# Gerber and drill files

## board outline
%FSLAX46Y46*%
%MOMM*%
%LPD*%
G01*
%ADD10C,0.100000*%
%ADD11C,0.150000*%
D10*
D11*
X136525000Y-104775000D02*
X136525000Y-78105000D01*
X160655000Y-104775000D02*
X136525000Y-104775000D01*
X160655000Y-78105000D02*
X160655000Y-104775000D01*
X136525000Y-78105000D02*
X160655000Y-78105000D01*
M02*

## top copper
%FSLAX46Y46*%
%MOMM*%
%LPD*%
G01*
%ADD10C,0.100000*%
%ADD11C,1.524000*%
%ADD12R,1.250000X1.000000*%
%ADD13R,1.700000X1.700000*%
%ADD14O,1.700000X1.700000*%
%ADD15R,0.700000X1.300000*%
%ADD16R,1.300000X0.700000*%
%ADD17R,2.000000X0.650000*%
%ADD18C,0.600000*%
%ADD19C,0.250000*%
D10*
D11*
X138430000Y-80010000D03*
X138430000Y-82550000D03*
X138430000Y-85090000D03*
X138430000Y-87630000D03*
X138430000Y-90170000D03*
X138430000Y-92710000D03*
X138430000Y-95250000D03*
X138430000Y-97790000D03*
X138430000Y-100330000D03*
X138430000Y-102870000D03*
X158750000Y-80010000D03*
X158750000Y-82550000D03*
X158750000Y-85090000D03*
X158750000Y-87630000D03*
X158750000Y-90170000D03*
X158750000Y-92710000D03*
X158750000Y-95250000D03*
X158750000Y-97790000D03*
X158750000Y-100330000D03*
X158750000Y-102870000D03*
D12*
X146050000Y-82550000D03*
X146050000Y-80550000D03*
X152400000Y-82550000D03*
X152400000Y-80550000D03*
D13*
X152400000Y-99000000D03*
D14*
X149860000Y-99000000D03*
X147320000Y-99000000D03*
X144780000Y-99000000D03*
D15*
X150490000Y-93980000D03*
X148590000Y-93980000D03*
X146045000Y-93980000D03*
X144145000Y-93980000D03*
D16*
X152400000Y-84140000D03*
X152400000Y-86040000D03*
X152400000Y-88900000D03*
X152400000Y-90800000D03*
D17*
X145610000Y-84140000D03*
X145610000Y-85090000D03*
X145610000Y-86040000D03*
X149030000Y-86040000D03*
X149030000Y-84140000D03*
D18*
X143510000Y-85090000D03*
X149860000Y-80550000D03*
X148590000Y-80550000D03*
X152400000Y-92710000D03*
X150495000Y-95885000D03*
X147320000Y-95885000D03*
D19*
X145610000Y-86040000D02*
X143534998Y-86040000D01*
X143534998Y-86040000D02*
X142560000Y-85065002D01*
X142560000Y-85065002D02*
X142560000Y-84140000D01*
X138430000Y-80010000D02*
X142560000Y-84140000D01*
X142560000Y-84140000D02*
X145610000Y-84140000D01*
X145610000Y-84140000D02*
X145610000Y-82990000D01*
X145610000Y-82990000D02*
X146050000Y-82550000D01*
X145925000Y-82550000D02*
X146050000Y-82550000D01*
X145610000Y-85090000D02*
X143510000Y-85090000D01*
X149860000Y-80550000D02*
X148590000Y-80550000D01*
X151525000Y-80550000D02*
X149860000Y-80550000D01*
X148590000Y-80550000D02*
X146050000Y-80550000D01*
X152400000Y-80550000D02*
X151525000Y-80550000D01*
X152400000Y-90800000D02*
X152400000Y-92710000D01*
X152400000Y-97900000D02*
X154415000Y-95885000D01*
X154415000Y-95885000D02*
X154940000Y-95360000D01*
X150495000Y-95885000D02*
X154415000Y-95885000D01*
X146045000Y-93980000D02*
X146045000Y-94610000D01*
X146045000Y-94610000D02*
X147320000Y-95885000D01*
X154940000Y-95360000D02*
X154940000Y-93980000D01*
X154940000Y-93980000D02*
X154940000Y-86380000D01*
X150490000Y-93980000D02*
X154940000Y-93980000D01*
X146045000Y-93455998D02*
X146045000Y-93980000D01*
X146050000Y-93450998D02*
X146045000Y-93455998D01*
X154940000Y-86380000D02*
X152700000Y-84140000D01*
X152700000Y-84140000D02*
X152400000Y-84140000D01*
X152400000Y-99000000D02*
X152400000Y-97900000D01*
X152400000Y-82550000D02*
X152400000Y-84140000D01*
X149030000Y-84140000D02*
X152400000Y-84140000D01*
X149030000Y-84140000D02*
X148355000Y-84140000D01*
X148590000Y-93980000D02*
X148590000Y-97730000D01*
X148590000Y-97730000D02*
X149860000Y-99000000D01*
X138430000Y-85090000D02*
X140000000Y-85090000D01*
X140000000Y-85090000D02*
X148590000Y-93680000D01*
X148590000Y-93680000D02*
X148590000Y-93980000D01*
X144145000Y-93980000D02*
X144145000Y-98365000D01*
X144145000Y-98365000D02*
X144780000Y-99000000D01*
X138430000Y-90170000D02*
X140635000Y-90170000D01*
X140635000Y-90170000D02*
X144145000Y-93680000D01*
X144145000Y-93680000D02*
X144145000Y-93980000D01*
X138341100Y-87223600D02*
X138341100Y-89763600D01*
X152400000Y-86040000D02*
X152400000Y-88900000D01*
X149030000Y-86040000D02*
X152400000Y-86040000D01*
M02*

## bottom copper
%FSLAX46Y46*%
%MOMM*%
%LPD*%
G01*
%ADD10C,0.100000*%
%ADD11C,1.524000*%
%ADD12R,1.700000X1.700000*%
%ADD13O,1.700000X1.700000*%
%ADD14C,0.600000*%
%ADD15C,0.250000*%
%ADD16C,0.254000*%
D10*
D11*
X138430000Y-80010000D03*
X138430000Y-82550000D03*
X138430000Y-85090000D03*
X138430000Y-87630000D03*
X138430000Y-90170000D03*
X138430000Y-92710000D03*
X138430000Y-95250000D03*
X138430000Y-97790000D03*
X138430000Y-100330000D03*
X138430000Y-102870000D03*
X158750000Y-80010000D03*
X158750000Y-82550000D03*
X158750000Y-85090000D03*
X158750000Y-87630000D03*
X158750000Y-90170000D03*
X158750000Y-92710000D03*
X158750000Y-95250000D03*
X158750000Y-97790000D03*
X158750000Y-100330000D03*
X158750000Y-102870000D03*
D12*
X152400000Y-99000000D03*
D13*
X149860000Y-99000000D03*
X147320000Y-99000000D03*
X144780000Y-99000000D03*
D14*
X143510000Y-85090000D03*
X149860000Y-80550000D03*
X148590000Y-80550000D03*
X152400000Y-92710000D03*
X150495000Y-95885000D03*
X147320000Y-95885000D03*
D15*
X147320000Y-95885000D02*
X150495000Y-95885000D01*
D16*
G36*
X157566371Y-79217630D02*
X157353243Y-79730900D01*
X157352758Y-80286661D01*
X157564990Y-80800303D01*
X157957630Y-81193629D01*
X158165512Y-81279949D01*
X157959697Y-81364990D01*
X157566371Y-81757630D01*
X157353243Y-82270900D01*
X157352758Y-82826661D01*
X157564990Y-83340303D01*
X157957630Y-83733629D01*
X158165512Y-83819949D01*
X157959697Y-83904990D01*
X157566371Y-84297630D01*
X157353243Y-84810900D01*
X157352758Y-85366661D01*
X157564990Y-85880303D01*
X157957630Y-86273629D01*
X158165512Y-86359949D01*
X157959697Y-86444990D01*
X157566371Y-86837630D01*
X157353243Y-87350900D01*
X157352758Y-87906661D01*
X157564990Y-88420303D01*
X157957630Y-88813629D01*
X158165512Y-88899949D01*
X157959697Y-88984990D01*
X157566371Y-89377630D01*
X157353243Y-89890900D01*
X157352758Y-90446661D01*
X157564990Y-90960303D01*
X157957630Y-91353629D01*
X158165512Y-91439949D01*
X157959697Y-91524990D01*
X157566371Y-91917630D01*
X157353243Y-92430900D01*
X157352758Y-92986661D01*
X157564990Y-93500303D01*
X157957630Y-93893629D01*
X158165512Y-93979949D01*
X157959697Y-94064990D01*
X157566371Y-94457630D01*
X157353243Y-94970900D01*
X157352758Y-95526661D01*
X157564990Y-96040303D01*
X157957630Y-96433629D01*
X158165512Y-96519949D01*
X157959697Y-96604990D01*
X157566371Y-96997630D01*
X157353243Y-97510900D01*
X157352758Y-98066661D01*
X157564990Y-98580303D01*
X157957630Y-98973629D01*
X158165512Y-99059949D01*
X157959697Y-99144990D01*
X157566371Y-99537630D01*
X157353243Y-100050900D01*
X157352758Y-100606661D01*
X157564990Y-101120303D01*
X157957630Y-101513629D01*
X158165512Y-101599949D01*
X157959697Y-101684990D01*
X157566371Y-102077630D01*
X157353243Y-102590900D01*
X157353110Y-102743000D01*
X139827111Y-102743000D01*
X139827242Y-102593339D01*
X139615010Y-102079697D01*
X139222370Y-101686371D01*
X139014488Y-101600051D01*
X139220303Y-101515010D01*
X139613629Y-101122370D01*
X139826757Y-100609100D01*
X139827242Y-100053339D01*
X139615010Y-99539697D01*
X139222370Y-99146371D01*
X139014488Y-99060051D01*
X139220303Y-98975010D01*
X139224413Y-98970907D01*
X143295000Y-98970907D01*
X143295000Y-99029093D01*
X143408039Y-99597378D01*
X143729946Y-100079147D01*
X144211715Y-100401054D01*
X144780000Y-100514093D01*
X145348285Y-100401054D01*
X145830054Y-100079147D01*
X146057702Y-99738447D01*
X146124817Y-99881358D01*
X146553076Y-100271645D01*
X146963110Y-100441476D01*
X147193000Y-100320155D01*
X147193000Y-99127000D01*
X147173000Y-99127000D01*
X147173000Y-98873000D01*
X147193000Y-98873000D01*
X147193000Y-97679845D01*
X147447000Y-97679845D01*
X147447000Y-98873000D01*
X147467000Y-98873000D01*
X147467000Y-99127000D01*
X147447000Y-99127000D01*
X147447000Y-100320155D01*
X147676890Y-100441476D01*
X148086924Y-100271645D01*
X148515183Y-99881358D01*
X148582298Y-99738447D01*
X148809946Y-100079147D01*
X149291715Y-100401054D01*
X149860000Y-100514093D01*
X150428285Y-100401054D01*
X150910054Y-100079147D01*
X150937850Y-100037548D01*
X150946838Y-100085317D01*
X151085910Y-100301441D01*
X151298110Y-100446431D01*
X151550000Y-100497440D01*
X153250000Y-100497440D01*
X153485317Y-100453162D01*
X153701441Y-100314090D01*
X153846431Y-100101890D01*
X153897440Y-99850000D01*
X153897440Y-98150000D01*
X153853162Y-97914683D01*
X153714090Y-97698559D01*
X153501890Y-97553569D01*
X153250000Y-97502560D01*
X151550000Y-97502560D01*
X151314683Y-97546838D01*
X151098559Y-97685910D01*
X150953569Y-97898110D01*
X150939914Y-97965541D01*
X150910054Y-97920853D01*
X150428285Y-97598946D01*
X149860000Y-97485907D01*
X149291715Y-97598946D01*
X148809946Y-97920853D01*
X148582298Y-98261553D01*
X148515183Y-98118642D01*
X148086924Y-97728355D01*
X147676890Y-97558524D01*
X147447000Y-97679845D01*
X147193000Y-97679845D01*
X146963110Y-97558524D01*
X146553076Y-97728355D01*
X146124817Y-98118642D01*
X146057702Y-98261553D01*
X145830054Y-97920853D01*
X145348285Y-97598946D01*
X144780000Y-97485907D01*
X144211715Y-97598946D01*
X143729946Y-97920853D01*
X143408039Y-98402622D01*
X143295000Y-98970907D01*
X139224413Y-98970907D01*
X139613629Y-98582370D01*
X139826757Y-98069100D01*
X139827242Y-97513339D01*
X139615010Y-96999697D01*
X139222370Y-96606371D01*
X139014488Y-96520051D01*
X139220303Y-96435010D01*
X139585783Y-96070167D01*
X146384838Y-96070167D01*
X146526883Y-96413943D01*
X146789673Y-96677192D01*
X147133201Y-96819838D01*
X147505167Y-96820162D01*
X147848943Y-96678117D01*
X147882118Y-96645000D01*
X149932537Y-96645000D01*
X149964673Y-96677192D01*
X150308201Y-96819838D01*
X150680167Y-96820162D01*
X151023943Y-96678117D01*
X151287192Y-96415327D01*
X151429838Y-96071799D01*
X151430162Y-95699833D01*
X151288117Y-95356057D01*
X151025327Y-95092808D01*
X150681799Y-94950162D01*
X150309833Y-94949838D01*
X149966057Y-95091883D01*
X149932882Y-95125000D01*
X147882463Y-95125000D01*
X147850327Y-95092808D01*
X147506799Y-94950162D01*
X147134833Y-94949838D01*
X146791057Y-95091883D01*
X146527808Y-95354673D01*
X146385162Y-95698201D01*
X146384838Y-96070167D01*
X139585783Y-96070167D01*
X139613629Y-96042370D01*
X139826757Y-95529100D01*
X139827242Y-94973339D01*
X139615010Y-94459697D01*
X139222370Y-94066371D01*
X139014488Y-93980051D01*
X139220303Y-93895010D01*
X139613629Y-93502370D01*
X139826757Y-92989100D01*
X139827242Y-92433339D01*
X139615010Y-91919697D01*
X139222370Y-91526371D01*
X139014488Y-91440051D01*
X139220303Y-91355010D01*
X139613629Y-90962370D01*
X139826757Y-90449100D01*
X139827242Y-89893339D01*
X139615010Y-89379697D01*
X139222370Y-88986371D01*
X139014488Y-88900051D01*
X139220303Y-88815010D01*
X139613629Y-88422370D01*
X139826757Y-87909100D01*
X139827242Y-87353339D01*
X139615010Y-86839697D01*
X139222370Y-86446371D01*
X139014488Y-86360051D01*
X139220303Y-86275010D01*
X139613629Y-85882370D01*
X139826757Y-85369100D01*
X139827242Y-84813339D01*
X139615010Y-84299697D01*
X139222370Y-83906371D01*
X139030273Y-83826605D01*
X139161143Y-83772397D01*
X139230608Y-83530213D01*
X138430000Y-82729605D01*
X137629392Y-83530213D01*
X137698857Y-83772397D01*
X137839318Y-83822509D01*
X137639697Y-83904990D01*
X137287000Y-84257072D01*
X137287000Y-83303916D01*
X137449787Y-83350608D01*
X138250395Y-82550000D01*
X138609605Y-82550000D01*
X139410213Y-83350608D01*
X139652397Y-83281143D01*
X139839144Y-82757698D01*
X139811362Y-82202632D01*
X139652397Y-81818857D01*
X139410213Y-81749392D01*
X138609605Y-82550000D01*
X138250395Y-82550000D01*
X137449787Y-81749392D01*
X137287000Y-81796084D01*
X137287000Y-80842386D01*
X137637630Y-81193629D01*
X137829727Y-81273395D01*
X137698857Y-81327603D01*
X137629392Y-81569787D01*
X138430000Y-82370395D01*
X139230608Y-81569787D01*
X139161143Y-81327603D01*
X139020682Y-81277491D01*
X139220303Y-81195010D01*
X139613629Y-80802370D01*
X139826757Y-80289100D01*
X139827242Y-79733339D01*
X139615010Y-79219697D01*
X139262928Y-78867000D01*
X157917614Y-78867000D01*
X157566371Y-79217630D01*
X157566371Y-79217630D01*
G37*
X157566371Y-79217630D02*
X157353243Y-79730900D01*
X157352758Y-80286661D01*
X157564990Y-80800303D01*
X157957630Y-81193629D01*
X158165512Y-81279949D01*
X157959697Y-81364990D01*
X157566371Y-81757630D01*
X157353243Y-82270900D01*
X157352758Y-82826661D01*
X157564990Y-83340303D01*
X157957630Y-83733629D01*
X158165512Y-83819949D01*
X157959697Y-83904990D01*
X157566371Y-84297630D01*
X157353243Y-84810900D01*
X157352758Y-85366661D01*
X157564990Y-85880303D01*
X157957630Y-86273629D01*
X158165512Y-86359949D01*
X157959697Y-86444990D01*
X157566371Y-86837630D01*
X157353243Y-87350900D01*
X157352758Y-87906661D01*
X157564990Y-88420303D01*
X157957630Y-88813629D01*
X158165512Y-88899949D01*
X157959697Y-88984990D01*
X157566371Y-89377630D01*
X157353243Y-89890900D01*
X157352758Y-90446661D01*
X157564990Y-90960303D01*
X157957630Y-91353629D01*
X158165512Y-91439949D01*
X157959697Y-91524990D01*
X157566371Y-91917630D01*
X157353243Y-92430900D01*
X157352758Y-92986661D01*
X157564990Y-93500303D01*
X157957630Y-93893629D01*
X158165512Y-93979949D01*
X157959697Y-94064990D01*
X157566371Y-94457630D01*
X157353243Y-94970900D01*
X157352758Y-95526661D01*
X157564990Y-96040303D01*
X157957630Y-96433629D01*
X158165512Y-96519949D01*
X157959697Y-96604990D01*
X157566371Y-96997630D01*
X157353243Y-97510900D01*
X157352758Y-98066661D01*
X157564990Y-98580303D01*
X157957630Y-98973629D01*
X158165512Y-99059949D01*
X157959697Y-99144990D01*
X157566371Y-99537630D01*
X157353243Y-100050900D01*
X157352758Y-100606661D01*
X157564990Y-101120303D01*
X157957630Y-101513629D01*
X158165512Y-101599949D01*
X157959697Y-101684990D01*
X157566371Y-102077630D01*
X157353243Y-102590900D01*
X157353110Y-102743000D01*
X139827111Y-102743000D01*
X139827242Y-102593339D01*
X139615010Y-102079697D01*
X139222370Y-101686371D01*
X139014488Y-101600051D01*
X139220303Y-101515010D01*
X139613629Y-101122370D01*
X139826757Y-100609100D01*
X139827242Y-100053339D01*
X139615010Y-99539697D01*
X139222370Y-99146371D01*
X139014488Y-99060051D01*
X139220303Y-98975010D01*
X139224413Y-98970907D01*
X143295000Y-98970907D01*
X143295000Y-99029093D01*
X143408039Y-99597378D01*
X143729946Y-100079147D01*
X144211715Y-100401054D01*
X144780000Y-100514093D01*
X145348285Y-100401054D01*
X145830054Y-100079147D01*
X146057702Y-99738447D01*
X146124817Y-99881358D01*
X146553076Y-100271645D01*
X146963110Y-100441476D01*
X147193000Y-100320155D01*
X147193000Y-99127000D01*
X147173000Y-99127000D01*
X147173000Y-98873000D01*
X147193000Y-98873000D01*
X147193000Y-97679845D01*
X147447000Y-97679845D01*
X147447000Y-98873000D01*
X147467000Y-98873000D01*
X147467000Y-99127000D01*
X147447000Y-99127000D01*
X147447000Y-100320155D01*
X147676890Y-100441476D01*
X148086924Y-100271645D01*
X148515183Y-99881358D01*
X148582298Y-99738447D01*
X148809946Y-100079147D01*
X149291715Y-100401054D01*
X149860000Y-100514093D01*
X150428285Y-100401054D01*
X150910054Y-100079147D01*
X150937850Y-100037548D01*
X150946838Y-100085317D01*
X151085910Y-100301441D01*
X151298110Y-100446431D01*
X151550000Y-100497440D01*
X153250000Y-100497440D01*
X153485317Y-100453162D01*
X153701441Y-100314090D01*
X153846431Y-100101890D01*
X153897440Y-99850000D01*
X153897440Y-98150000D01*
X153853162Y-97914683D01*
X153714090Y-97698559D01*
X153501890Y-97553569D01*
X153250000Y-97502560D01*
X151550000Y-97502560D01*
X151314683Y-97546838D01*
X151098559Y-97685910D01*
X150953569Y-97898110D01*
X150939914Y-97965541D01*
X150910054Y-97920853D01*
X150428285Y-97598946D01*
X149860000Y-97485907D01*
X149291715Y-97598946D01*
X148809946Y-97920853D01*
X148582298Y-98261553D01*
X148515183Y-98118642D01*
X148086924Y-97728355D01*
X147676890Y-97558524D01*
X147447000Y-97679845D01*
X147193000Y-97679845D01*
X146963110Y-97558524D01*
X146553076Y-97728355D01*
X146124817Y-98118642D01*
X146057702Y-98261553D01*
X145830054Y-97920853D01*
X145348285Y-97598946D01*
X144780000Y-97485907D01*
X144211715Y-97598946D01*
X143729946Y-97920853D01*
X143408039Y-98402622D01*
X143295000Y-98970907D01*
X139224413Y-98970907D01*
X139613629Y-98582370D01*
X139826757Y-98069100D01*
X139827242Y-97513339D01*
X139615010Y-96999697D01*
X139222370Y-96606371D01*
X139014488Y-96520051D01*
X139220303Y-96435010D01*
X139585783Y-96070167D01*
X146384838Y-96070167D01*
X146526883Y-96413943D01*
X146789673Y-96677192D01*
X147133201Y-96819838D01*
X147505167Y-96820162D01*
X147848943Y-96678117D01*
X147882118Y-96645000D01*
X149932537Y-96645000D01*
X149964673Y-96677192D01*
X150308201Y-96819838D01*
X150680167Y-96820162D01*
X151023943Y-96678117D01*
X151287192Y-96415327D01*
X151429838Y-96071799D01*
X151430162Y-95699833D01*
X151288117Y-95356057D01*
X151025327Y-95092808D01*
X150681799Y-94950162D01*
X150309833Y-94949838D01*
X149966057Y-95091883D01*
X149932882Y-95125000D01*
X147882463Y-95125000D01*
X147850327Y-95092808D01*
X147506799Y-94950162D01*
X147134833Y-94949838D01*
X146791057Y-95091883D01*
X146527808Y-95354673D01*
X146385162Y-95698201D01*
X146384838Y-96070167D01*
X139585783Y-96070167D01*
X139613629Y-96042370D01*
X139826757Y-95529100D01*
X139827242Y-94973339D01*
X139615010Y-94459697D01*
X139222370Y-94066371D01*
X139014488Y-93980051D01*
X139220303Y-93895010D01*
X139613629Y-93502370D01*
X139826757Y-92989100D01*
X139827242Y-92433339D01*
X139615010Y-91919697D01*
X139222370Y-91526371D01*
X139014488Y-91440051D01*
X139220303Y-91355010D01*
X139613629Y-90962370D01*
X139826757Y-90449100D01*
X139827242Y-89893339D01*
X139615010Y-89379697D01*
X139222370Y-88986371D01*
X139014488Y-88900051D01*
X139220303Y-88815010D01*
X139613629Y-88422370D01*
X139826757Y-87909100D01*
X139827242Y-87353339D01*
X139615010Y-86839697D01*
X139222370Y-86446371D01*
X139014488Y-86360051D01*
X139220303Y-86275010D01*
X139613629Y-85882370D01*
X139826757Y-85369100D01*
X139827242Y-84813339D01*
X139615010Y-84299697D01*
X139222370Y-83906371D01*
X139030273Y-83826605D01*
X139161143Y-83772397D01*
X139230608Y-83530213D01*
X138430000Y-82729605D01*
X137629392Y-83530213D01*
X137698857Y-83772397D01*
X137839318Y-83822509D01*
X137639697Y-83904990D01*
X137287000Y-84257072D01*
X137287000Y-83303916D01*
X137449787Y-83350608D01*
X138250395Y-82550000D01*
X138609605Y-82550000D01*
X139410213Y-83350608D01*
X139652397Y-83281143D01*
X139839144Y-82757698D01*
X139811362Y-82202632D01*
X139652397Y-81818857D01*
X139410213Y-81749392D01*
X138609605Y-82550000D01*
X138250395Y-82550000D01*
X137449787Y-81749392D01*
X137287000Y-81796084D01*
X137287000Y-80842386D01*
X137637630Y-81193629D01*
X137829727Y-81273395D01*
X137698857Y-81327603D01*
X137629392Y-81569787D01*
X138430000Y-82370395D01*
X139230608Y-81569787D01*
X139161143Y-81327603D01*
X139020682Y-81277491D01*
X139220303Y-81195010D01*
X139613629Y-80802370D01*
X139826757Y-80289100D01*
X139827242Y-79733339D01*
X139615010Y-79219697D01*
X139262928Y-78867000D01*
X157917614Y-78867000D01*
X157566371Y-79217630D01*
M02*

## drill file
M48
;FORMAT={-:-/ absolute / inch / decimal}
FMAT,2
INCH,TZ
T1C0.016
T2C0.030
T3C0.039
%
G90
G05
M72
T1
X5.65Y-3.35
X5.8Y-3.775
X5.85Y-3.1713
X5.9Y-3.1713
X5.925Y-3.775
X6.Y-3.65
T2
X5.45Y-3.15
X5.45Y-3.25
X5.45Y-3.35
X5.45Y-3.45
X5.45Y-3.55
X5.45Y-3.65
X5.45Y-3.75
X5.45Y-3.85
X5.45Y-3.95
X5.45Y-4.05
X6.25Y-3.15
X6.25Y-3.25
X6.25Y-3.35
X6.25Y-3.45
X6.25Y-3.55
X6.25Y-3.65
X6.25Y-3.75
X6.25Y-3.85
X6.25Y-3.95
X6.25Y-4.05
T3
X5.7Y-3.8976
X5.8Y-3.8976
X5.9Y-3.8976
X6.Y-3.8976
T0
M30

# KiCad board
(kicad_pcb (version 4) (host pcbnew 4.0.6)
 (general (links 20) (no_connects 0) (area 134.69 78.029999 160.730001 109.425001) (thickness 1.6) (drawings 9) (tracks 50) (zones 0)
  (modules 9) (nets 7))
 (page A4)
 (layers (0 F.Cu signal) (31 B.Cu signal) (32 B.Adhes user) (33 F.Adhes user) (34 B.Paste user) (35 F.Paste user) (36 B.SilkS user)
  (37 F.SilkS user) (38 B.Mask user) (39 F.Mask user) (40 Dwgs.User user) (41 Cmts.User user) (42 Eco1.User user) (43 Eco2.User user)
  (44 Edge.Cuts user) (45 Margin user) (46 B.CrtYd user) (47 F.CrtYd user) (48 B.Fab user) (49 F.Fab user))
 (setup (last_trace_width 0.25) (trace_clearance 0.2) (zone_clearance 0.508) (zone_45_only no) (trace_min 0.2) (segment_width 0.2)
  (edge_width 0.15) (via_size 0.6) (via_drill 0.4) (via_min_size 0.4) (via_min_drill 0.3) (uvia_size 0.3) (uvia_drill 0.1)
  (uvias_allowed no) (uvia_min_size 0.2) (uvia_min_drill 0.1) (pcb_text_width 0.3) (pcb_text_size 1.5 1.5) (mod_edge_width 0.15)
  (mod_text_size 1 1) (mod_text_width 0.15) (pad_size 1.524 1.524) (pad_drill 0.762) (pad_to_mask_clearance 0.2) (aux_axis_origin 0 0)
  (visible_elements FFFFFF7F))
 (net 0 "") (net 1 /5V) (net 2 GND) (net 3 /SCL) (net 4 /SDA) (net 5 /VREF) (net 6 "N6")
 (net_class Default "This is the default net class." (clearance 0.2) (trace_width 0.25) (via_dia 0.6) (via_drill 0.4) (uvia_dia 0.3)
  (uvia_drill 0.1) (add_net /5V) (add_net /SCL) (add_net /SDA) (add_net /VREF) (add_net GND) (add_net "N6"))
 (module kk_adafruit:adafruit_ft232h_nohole (layer F.Cu) (at 148.59 105.41)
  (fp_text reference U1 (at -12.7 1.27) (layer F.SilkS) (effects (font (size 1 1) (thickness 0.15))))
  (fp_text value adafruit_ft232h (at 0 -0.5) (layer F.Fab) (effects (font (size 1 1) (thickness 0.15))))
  (pad 1 thru_hole circle (at -10.16 -25.4) (size 1.524 1.524) (drill 0.762) (layers *.Cu *.Mask) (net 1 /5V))
  (pad 2 thru_hole circle (at -10.16 -22.86) (size 1.524 1.524) (drill 0.762) (layers *.Cu *.Mask) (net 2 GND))
  (pad 3 thru_hole circle (at -10.16 -20.32) (size 1.524 1.524) (drill 0.762) (layers *.Cu *.Mask) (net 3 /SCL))
  (pad 4 thru_hole circle (at -10.16 -17.78) (size 1.524 1.524) (drill 0.762) (layers *.Cu *.Mask) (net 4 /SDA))
  (pad 5 thru_hole circle (at -10.16 -15.24) (size 1.524 1.524) (drill 0.762) (layers *.Cu *.Mask) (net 4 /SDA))
  (pad 6 thru_hole circle (at -10.16 -12.7) (size 1.524 1.524) (drill 0.762) (layers *.Cu *.Mask))
  (pad 7 thru_hole circle (at -10.16 -10.16) (size 1.524 1.524) (drill 0.762) (layers *.Cu *.Mask))
  (pad 8 thru_hole circle (at -10.16 -7.62) (size 1.524 1.524) (drill 0.762) (layers *.Cu *.Mask))
  (pad 9 thru_hole circle (at -10.16 -5.08) (size 1.524 1.524) (drill 0.762) (layers *.Cu *.Mask))
  (pad 10 thru_hole circle (at -10.16 -2.54) (size 1.524 1.524) (drill 0.762) (layers *.Cu *.Mask))
  (pad 20 thru_hole circle (at 10.16 -25.4) (size 1.524 1.524) (drill 0.762) (layers *.Cu *.Mask))
  (pad 19 thru_hole circle (at 10.16 -22.86) (size 1.524 1.524) (drill 0.762) (layers *.Cu *.Mask))
  (pad 18 thru_hole circle (at 10.16 -20.32) (size 1.524 1.524) (drill 0.762) (layers *.Cu *.Mask))
  (pad 17 thru_hole circle (at 10.16 -17.78) (size 1.524 1.524) (drill 0.762) (layers *.Cu *.Mask))
  (pad 16 thru_hole circle (at 10.16 -15.24) (size 1.524 1.524) (drill 0.762) (layers *.Cu *.Mask))
  (pad 15 thru_hole circle (at 10.16 -12.7) (size 1.524 1.524) (drill 0.762) (layers *.Cu *.Mask))
  (pad 14 thru_hole circle (at 10.16 -10.16) (size 1.524 1.524) (drill 0.762) (layers *.Cu *.Mask))
  (pad 13 thru_hole circle (at 10.16 -7.62) (size 1.524 1.524) (drill 0.762) (layers *.Cu *.Mask))
  (pad 12 thru_hole circle (at 10.16 -5.08) (size 1.524 1.524) (drill 0.762) (layers *.Cu *.Mask))
  (pad 11 thru_hole circle (at 10.16 -2.54) (size 1.524 1.524) (drill 0.762) (layers *.Cu *.Mask)))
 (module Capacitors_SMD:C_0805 (layer F.Cu) (at 146.05 81.55 90)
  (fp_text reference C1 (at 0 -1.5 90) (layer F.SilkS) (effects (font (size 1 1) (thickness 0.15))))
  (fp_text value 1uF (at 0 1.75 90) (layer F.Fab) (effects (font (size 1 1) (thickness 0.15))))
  (pad 1 smd rect (at -1 0 90) (size 1 1.25) (layers F.Cu F.Paste F.Mask) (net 1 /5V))
  (pad 2 smd rect (at 1 0 90) (size 1 1.25) (layers F.Cu F.Paste F.Mask) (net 2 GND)))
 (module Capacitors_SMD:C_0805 (layer F.Cu) (at 152.4 81.55 90)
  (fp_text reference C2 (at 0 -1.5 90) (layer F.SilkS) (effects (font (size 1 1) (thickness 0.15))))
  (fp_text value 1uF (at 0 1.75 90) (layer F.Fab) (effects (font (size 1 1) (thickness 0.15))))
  (pad 1 smd rect (at -1 0 90) (size 1 1.25) (layers F.Cu F.Paste F.Mask) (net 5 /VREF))
  (pad 2 smd rect (at 1 0 90) (size 1 1.25) (layers F.Cu F.Paste F.Mask) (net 2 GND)))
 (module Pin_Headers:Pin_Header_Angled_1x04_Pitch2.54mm (layer F.Cu) (at 152.4 99 270)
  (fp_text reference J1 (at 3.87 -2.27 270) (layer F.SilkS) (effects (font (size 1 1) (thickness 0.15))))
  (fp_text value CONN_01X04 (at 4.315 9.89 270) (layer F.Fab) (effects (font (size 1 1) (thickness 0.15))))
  (pad 1 thru_hole rect (at 0 0 270) (size 1.7 1.7) (drill 1) (layers *.Cu *.Mask) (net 5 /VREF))
  (pad 2 thru_hole oval (at 0 2.54 270) (size 1.7 1.7) (drill 1) (layers *.Cu *.Mask) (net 3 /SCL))
  (pad 3 thru_hole oval (at 0 5.08 270) (size 1.7 1.7) (drill 1) (layers *.Cu *.Mask) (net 2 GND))
  (pad 4 thru_hole oval (at 0 7.62 270) (size 1.7 1.7) (drill 1) (layers *.Cu *.Mask) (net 4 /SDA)))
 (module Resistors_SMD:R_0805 (layer F.Cu) (at 149.54 93.98 180)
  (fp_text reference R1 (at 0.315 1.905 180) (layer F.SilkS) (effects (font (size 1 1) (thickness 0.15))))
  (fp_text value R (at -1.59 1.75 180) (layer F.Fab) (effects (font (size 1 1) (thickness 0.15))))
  (pad 1 smd rect (at -0.95 0 180) (size 0.7 1.3) (layers F.Cu F.Paste F.Mask) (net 5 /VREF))
  (pad 2 smd rect (at 0.95 0 180) (size 0.7 1.3) (layers F.Cu F.Paste F.Mask) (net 3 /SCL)))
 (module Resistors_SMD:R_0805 (layer F.Cu) (at 145.095 93.98 180)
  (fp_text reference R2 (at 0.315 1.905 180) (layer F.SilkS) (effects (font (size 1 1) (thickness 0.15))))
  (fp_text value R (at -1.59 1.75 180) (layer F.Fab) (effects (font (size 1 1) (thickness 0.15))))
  (pad 1 smd rect (at -0.95 0 180) (size 0.7 1.3) (layers F.Cu F.Paste F.Mask) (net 5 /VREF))
  (pad 2 smd rect (at 0.95 0 180) (size 0.7 1.3) (layers F.Cu F.Paste F.Mask) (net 4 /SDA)))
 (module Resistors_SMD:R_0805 (layer F.Cu) (at 152.4 85.09 270)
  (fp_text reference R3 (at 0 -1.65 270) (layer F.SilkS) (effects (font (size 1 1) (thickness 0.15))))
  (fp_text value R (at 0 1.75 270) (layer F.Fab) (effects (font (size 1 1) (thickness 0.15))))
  (pad 1 smd rect (at -0.95 0 270) (size 0.7 1.3) (layers F.Cu F.Paste F.Mask) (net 5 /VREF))
  (pad 2 smd rect (at 0.95 0 270) (size 0.7 1.3) (layers F.Cu F.Paste F.Mask) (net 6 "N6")))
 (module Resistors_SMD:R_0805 (layer F.Cu) (at 152.4 89.85 270)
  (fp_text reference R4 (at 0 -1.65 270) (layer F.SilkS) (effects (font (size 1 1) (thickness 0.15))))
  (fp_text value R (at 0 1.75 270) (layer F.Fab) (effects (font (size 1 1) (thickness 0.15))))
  (pad 1 smd rect (at -0.95 0 270) (size 0.7 1.3) (layers F.Cu F.Paste F.Mask) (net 6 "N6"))
  (pad 2 smd rect (at 0.95 0 270) (size 0.7 1.3) (layers F.Cu F.Paste F.Mask) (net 2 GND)))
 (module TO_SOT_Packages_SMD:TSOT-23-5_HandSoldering (layer F.Cu) (at 147.32 85.09)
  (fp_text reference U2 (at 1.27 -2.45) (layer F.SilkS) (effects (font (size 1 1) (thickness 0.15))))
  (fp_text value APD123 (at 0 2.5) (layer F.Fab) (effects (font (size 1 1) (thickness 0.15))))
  (pad 1 smd rect (at -1.71 -0.95) (size 2 0.65) (layers F.Cu F.Paste F.Mask) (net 1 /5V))
  (pad 2 smd rect (at -1.71 0) (size 2 0.65) (layers F.Cu F.Paste F.Mask) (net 2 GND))
  (pad 3 smd rect (at -1.71 0.95) (size 2 0.65) (layers F.Cu F.Paste F.Mask) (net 1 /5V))
  (pad 4 smd rect (at 1.71 0.95) (size 2 0.65) (layers F.Cu F.Paste F.Mask) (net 6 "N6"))
  (pad 5 smd rect (at 1.71 -0.95) (size 2 0.65) (layers F.Cu F.Paste F.Mask) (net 5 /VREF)))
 (gr_line (start 136.525 104.775) (end 136.525 78.105) (layer Edge.Cuts) (width 0.15))
 (gr_line (start 160.655 104.775) (end 136.525 104.775) (layer Edge.Cuts) (width 0.15))
 (gr_line (start 160.655 78.105) (end 160.655 104.775) (layer Edge.Cuts) (width 0.15))
 (gr_line (start 136.525 78.105) (end 160.655 78.105) (layer Edge.Cuts) (width 0.15))
 (segment (start 145.61 86.04) (end 143.534998 86.04) (width 0.25) (layer F.Cu) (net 1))
 (segment (start 143.534998 86.04) (end 142.56 85.065002) (width 0.25) (layer F.Cu) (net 1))
 (segment (start 142.56 85.065002) (end 142.56 84.14) (width 0.25) (layer F.Cu) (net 1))
 (segment (start 138.43 80.01) (end 142.56 84.14) (width 0.25) (layer F.Cu) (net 1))
 (segment (start 142.56 84.14) (end 145.61 84.14) (width 0.25) (layer F.Cu) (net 1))
 (segment (start 145.61 84.14) (end 145.61 82.99) (width 0.25) (layer F.Cu) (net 1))
 (segment (start 145.61 82.99) (end 146.05 82.55) (width 0.25) (layer F.Cu) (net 1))
 (segment (start 145.925 82.55) (end 146.05 82.55) (width 0.25) (layer F.Cu) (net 1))
 (segment (start 145.61 85.09) (end 143.51 85.09) (width 0.25) (layer F.Cu) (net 2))
 (via (at 143.51 85.09) (size 0.6) (drill 0.4) (layers F.Cu B.Cu) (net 2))
 (segment (start 149.86 80.55) (end 148.59 80.55) (width 0.25) (layer F.Cu) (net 2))
 (segment (start 151.525 80.55) (end 149.86 80.55) (width 0.25) (layer F.Cu) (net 2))
 (via (at 149.86 80.55) (size 0.6) (drill 0.4) (layers F.Cu B.Cu) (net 2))
 (segment (start 148.59 80.55) (end 146.05 80.55) (width 0.25) (layer F.Cu) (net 2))
 (via (at 148.59 80.55) (size 0.6) (drill 0.4) (layers F.Cu B.Cu) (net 2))
 (segment (start 152.4 80.55) (end 151.525 80.55) (width 0.25) (layer F.Cu) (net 2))
 (segment (start 152.4 90.8) (end 152.4 92.71) (width 0.25) (layer F.Cu) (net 2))
 (via (at 152.4 92.71) (size 0.6) (drill 0.4) (layers F.Cu B.Cu) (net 2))
 (segment (start 152.4 97.9) (end 154.415 95.885) (width 0.25) (layer F.Cu) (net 5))
 (segment (start 154.415 95.885) (end 154.94 95.36) (width 0.25) (layer F.Cu) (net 5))
 (segment (start 150.495 95.885) (end 154.415 95.885) (width 0.25) (layer F.Cu) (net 5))
 (segment (start 147.32 95.885) (end 150.495 95.885) (width 0.25) (layer B.Cu) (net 5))
 (via (at 150.495 95.885) (size 0.6) (drill 0.4) (layers F.Cu B.Cu) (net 5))
 (segment (start 146.045 93.98) (end 146.045 94.61) (width 0.25) (layer F.Cu) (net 5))
 (segment (start 146.045 94.61) (end 147.32 95.885) (width 0.25) (layer F.Cu) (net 5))
 (via (at 147.32 95.885) (size 0.6) (drill 0.4) (layers F.Cu B.Cu) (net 5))
 (segment (start 154.94 95.36) (end 154.94 93.98) (width 0.25) (layer F.Cu) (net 5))
 (segment (start 154.94 93.98) (end 154.94 86.38) (width 0.25) (layer F.Cu) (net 5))
 (segment (start 150.49 93.98) (end 154.94 93.98) (width 0.25) (layer F.Cu) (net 5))
 (segment (start 146.045 93.455998) (end 146.045 93.98) (width 0.25) (layer F.Cu) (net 5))
 (segment (start 146.05 93.450998) (end 146.045 93.455998) (width 0.25) (layer F.Cu) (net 5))
 (segment (start 154.94 86.38) (end 152.7 84.14) (width 0.25) (layer F.Cu) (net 5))
 (segment (start 152.7 84.14) (end 152.4 84.14) (width 0.25) (layer F.Cu) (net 5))
 (segment (start 152.4 99) (end 152.4 97.9) (width 0.25) (layer F.Cu) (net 5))
 (segment (start 152.4 82.55) (end 152.4 84.14) (width 0.25) (layer F.Cu) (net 5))
 (segment (start 149.03 84.14) (end 152.4 84.14) (width 0.25) (layer F.Cu) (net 5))
 (segment (start 149.03 84.14) (end 148.355 84.14) (width 0.25) (layer F.Cu) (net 5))
 (segment (start 148.59 93.98) (end 148.59 97.73) (width 0.25) (layer F.Cu) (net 3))
 (segment (start 148.59 97.73) (end 149.86 99) (width 0.25) (layer F.Cu) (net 3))
 (segment (start 138.43 85.09) (end 140 85.09) (width 0.25) (layer F.Cu) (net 3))
 (segment (start 140 85.09) (end 148.59 93.68) (width 0.25) (layer F.Cu) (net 3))
 (segment (start 148.59 93.68) (end 148.59 93.98) (width 0.25) (layer F.Cu) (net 3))
 (segment (start 144.145 93.98) (end 144.145 98.365) (width 0.25) (layer F.Cu) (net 4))
 (segment (start 144.145 98.365) (end 144.78 99) (width 0.25) (layer F.Cu) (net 4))
 (segment (start 138.43 90.17) (end 140.635 90.17) (width 0.25) (layer F.Cu) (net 4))
 (segment (start 140.635 90.17) (end 144.145 93.68) (width 0.25) (layer F.Cu) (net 4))
 (segment (start 144.145 93.68) (end 144.145 93.98) (width 0.25) (layer F.Cu) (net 4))
 (segment (start 138.3411 87.2236) (end 138.3411 89.7636) (width 0.25) (layer F.Cu) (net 4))
 (segment (start 152.4 86.04) (end 152.4 88.9) (width 0.25) (layer F.Cu) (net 6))
 (segment (start 149.03 86.04) (end 152.4 86.04) (width 0.25) (layer F.Cu) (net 6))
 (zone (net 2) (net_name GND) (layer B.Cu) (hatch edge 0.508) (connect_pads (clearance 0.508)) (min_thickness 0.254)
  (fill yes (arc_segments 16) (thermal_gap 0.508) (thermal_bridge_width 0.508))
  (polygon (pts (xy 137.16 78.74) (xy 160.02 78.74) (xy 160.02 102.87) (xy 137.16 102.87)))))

